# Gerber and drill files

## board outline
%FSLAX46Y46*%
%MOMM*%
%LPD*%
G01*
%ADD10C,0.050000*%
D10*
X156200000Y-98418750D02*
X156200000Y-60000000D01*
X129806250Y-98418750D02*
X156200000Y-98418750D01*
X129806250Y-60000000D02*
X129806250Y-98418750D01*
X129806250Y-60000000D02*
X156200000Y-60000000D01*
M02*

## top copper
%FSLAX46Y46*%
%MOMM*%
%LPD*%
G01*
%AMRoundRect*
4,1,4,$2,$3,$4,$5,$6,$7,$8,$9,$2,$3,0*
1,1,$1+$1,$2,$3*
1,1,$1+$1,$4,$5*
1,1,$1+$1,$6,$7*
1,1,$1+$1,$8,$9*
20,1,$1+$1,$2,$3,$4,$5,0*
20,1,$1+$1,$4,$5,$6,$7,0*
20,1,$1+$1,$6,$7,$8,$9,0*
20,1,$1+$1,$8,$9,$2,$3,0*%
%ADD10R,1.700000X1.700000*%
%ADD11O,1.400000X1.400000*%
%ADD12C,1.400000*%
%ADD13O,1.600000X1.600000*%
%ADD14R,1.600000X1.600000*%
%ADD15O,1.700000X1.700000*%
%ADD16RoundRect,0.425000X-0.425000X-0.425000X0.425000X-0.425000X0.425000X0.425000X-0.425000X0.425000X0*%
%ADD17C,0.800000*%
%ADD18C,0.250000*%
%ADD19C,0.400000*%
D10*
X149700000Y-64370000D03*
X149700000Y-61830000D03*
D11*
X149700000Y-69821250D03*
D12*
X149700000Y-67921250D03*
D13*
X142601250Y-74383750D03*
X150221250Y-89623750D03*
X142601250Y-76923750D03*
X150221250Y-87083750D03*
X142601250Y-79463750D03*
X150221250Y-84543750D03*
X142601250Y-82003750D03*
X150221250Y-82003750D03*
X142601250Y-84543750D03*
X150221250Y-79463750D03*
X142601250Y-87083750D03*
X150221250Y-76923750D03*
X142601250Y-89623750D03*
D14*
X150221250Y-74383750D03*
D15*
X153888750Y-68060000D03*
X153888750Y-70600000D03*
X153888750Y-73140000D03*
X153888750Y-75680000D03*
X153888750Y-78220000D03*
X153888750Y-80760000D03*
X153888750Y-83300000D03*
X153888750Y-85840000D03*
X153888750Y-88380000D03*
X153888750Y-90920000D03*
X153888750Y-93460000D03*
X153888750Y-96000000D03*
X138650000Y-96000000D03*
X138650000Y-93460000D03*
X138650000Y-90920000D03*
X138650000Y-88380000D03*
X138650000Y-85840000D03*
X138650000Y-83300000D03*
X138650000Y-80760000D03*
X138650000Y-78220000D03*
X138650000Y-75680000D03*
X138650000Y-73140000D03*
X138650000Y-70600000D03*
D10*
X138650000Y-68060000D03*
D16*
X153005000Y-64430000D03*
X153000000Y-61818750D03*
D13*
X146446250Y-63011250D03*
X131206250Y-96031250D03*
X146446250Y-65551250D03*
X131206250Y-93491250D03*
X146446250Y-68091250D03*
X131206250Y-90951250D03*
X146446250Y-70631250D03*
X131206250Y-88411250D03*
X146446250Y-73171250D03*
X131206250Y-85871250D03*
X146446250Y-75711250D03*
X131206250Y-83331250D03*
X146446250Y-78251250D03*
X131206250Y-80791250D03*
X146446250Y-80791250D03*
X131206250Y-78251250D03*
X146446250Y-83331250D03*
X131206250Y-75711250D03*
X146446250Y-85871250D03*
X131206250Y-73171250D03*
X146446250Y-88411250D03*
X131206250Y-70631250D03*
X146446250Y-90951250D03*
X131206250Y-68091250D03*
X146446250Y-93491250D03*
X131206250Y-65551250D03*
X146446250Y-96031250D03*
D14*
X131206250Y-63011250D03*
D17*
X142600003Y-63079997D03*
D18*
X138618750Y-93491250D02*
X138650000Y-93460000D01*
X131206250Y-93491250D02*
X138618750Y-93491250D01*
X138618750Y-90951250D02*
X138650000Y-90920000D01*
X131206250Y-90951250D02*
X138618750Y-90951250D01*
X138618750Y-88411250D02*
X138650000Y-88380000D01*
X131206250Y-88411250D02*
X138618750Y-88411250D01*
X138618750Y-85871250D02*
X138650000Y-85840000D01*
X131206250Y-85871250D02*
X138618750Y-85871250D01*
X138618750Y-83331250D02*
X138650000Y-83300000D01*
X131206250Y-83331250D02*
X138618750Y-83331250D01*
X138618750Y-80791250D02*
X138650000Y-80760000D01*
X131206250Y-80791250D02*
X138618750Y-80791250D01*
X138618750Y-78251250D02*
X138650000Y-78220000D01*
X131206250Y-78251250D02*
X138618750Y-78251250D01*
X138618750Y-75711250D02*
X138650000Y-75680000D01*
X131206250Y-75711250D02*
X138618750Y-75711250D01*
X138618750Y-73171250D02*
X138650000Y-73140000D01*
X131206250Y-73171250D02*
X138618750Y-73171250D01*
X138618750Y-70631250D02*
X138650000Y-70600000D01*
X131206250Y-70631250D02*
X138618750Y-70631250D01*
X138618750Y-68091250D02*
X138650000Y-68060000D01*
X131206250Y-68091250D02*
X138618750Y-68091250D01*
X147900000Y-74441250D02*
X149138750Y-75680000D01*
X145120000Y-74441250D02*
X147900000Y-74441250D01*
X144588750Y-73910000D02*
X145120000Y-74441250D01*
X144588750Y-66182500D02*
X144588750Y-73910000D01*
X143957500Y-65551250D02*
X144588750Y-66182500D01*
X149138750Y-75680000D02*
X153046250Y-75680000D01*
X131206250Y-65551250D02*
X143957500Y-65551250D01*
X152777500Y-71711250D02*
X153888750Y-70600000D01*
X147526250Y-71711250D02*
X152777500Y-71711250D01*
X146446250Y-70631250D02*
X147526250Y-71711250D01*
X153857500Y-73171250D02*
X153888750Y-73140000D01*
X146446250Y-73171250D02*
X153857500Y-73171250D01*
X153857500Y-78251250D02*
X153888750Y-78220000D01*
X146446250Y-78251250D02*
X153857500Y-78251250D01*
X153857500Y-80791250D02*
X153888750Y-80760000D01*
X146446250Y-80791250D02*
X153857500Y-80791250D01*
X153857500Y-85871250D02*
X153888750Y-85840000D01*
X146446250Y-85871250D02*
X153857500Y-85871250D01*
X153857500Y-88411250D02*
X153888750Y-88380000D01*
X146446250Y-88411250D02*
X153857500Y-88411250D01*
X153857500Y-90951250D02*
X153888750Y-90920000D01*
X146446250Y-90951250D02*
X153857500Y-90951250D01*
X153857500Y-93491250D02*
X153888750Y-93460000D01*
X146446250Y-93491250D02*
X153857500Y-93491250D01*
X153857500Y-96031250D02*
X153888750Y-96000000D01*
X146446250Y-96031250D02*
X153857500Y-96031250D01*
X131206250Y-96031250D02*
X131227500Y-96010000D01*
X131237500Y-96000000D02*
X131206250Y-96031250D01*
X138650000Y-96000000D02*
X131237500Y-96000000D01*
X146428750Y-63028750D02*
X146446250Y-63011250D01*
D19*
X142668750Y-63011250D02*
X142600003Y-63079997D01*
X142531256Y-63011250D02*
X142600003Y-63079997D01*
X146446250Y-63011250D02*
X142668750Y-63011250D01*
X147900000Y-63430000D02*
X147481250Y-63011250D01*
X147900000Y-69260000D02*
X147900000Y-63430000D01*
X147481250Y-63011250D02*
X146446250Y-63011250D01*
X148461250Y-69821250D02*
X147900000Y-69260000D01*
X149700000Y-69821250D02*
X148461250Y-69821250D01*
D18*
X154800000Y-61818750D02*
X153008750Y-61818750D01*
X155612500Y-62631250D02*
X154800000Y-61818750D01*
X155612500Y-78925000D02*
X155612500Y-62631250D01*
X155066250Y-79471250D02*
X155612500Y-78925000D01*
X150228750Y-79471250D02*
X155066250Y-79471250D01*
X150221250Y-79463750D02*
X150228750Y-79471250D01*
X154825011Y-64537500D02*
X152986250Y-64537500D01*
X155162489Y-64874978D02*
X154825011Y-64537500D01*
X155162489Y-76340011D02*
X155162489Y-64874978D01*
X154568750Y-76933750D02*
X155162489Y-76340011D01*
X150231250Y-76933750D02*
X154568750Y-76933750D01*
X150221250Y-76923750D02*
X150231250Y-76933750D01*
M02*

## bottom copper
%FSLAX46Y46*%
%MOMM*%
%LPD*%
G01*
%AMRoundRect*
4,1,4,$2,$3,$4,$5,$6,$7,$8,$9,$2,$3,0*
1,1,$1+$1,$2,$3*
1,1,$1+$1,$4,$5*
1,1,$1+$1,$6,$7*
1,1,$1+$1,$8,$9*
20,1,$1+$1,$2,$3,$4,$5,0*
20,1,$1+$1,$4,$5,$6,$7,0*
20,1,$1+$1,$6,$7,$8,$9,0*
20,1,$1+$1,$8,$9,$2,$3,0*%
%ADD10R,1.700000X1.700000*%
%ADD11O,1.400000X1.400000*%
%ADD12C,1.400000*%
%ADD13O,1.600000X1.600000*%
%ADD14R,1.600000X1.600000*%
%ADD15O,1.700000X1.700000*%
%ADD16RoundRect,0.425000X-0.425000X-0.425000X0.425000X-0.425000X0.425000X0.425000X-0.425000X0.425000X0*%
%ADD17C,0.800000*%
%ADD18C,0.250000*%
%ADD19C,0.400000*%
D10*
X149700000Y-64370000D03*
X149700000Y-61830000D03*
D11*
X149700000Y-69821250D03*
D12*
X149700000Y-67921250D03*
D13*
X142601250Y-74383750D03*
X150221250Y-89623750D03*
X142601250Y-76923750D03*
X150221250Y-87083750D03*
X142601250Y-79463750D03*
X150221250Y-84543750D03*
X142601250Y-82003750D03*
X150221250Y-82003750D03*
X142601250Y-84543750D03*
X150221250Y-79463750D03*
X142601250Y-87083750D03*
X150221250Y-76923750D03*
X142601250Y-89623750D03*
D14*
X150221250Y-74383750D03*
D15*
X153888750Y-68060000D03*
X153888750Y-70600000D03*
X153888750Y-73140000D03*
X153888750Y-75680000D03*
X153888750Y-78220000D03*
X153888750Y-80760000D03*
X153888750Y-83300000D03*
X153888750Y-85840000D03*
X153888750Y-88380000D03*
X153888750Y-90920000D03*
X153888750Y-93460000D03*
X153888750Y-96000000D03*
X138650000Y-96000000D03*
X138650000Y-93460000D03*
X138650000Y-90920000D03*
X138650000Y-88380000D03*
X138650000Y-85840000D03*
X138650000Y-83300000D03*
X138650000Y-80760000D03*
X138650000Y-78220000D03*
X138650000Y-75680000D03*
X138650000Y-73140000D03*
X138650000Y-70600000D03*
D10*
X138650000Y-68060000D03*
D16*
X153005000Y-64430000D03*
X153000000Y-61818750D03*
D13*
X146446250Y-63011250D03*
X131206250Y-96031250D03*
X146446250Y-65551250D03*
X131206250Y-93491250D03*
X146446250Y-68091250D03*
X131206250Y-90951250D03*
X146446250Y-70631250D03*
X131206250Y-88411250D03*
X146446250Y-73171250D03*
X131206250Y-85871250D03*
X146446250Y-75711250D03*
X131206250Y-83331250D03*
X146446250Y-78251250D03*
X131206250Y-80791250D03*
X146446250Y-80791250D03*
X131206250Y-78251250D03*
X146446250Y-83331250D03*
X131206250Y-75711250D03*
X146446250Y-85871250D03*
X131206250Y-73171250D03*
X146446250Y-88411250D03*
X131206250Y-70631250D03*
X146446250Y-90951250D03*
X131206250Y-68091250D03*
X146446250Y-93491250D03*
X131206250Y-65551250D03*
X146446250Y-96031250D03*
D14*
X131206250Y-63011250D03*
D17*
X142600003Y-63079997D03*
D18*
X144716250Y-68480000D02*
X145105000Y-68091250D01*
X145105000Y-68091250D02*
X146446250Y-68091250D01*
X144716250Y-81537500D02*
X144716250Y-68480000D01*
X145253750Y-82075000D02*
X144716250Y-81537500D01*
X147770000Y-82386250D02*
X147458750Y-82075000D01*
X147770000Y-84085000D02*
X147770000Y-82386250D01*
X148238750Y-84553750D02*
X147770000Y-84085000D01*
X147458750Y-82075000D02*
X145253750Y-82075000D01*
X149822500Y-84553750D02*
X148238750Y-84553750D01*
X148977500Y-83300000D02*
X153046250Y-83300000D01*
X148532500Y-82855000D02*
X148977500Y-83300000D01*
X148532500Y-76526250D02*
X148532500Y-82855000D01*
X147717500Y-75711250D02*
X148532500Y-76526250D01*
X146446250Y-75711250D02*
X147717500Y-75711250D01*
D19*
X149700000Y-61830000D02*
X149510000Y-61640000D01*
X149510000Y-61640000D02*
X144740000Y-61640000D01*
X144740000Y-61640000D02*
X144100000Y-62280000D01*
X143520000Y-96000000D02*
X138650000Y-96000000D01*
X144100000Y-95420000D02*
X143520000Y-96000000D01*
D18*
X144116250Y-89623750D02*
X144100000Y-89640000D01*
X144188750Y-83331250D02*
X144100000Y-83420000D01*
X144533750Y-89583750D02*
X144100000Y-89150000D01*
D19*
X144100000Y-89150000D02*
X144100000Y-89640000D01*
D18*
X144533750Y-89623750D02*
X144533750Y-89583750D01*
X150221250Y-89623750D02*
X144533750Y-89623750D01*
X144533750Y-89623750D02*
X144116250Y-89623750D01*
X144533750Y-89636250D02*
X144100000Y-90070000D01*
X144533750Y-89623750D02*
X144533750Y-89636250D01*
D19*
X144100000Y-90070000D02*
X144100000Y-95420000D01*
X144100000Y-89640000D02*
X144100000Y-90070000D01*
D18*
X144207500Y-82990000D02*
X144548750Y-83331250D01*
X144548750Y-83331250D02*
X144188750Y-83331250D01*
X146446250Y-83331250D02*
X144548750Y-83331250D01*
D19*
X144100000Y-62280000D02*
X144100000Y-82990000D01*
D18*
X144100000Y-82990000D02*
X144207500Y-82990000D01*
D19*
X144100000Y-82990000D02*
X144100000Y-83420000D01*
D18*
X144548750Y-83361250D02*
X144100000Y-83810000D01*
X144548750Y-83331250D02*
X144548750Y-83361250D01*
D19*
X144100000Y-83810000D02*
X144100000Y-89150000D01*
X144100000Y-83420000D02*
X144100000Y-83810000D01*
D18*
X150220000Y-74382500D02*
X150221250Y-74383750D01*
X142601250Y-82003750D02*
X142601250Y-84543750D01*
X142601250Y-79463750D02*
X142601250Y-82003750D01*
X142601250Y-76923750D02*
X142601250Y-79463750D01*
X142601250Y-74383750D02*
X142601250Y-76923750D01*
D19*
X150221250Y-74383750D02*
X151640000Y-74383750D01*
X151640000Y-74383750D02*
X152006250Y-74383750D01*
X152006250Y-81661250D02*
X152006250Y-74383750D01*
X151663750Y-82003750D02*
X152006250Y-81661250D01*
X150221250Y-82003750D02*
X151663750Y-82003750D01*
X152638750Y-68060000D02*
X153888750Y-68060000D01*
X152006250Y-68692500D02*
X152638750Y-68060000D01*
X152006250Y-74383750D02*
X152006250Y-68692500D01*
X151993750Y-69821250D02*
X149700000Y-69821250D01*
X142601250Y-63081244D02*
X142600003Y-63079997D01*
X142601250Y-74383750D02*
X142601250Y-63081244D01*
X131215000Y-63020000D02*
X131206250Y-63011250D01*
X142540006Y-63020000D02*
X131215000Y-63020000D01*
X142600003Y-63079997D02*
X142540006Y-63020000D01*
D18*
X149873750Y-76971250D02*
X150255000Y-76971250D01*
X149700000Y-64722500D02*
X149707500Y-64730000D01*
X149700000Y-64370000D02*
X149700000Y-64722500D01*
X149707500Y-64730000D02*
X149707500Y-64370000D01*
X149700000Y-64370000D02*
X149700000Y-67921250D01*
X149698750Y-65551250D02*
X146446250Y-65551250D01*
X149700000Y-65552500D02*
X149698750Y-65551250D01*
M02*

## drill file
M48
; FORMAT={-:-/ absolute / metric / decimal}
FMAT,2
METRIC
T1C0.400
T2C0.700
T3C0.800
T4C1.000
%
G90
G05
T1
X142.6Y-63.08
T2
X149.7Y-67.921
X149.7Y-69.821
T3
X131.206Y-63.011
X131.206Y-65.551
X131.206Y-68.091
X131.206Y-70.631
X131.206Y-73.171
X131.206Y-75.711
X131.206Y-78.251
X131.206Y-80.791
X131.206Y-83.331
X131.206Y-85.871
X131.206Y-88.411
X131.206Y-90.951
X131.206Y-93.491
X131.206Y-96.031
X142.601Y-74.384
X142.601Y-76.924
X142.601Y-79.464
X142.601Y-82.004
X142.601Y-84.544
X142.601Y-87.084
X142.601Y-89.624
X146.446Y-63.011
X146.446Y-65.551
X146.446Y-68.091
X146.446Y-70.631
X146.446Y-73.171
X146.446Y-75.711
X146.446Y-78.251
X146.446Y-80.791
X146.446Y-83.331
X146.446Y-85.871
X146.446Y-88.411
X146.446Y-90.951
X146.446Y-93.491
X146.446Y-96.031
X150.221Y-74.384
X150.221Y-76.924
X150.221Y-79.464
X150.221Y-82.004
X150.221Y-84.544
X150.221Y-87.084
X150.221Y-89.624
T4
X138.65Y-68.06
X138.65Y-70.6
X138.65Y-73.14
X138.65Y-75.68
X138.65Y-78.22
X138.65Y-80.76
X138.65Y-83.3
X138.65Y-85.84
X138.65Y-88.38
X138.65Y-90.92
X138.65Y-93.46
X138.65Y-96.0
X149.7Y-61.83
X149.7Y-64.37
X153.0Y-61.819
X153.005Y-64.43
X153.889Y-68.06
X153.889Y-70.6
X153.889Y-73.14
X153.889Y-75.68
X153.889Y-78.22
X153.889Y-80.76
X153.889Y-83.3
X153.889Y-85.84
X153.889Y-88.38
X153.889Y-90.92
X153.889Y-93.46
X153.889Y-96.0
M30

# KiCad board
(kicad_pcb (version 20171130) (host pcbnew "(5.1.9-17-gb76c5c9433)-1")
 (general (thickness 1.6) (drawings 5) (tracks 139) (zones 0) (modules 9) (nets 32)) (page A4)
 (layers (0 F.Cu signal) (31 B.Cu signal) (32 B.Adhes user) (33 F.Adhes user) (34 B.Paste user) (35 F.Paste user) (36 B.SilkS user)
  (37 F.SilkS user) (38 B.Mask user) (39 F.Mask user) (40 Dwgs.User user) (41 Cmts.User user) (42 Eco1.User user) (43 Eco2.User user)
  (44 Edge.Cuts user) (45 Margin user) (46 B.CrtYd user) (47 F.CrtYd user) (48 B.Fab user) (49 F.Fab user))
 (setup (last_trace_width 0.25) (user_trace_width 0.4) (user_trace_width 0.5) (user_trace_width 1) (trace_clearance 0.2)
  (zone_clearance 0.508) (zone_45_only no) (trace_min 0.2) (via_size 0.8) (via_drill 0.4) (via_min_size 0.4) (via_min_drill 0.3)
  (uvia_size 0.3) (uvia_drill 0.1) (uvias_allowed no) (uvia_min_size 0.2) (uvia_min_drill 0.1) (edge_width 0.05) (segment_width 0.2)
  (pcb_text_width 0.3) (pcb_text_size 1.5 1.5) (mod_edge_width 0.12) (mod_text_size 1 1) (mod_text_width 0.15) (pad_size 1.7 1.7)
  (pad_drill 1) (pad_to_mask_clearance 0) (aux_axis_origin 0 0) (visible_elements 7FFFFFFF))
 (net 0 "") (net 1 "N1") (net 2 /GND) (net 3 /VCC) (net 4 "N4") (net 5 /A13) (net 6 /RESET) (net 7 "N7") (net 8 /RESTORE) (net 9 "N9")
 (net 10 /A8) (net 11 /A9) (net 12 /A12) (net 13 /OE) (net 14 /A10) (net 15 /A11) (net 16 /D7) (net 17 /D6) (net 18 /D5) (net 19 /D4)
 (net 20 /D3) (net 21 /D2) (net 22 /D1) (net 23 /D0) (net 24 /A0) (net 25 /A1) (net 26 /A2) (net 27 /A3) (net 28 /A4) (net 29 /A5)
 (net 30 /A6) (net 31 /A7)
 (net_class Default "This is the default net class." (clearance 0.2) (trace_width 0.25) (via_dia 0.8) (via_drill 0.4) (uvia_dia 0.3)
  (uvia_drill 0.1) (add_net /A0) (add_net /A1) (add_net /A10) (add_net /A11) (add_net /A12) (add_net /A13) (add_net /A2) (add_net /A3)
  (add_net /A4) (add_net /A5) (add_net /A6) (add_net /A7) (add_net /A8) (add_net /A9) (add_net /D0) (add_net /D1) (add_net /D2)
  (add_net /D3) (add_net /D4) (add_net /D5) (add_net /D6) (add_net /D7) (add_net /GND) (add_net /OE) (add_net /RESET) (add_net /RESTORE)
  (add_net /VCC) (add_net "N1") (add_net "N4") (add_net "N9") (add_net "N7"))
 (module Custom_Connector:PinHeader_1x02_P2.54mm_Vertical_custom (layer F.Cu) (at 149.7 61.83)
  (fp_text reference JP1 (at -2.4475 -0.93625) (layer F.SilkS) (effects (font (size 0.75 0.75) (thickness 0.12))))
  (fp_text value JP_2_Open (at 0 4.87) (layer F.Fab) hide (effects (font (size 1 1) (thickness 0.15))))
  (pad 2 thru_hole rect (at 0 2.54) (size 1.7 1.7) (drill 1) (layers *.Cu *.Mask) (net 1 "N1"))
  (pad 1 thru_hole rect (at 0 0) (size 1.7 1.7) (drill 1) (layers *.Cu *.Mask) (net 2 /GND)))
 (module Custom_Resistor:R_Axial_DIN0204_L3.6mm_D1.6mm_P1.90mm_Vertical (layer F.Cu) (at 149.7 67.92125 270)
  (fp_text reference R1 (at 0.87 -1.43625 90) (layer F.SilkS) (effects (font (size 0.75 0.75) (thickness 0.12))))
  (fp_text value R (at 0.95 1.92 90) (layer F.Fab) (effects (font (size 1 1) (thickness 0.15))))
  (pad 2 thru_hole oval (at 1.9 0 270) (size 1.4 1.4) (drill 0.7) (layers *.Cu *.Mask) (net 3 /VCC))
  (pad 1 thru_hole circle (at 0 0 270) (size 1.4 1.4) (drill 0.7) (layers *.Cu *.Mask) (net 1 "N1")))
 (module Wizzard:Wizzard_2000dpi (layer F.Cu) (at 138.17125 65.0425 350)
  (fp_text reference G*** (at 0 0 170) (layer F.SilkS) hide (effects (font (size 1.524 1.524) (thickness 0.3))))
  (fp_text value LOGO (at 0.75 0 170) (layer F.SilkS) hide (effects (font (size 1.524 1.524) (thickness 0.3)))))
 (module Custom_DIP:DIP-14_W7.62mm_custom (layer B.Cu) (at 150.22125 74.38375 180)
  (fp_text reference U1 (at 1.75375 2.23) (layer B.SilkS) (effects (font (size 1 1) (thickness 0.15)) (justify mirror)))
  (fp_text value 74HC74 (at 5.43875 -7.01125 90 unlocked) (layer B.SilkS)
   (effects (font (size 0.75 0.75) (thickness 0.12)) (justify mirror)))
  (pad 14 thru_hole oval (at 7.62 0 180) (size 1.6 1.6) (drill 0.8) (layers *.Cu *.Mask) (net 3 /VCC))
  (pad 7 thru_hole oval (at 0 -15.24 180) (size 1.6 1.6) (drill 0.8) (layers *.Cu *.Mask) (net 2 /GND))
  (pad 13 thru_hole oval (at 7.62 -2.54 180) (size 1.6 1.6) (drill 0.8) (layers *.Cu *.Mask) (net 3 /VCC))
  (pad 6 thru_hole oval (at 0 -12.7 180) (size 1.6 1.6) (drill 0.8) (layers *.Cu *.Mask) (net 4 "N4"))
  (pad 12 thru_hole oval (at 7.62 -5.08 180) (size 1.6 1.6) (drill 0.8) (layers *.Cu *.Mask) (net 3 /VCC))
  (pad 5 thru_hole oval (at 0 -10.16 180) (size 1.6 1.6) (drill 0.8) (layers *.Cu *.Mask) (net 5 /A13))
  (pad 11 thru_hole oval (at 7.62 -7.62 180) (size 1.6 1.6) (drill 0.8) (layers *.Cu *.Mask) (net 3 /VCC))
  (pad 4 thru_hole oval (at 0 -7.62 180) (size 1.6 1.6) (drill 0.8) (layers *.Cu *.Mask) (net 3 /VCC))
  (pad 10 thru_hole oval (at 7.62 -10.16 180) (size 1.6 1.6) (drill 0.8) (layers *.Cu *.Mask) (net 3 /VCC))
  (pad 3 thru_hole oval (at 0 -5.08 180) (size 1.6 1.6) (drill 0.8) (layers *.Cu *.Mask) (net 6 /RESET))
  (pad 9 thru_hole oval (at 7.62 -12.7 180) (size 1.6 1.6) (drill 0.8) (layers *.Cu *.Mask) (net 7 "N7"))
  (pad 2 thru_hole oval (at 0 -2.54 180) (size 1.6 1.6) (drill 0.8) (layers *.Cu *.Mask) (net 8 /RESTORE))
  (pad 8 thru_hole oval (at 7.62 -15.24 180) (size 1.6 1.6) (drill 0.8) (layers *.Cu *.Mask) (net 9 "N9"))
  (pad 1 thru_hole rect (at 0 0 180) (size 1.6 1.6) (drill 0.8) (layers *.Cu *.Mask) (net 3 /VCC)))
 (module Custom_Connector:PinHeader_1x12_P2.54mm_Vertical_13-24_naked (layer F.Cu) (at 153.88875 68.06)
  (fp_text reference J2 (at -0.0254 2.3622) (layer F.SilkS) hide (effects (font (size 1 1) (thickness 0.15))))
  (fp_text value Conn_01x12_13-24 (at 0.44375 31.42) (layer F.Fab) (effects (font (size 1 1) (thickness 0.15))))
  (pad 24 thru_hole oval (at 0 0) (size 1.7 1.7) (drill 1) (layers *.Cu *.Mask) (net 3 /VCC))
  (pad 23 thru_hole oval (at 0 2.54) (size 1.7 1.7) (drill 1) (layers *.Cu *.Mask) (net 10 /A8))
  (pad 22 thru_hole oval (at 0 5.08) (size 1.7 1.7) (drill 1) (layers *.Cu *.Mask) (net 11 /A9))
  (pad 21 thru_hole oval (at 0 7.62) (size 1.7 1.7) (drill 1) (layers *.Cu *.Mask) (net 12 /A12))
  (pad 20 thru_hole oval (at 0 10.16) (size 1.7 1.7) (drill 1) (layers *.Cu *.Mask) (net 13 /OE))
  (pad 19 thru_hole oval (at 0 12.7) (size 1.7 1.7) (drill 1) (layers *.Cu *.Mask) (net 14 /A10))
  (pad 18 thru_hole oval (at 0 15.24) (size 1.7 1.7) (drill 1) (layers *.Cu *.Mask) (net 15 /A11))
  (pad 17 thru_hole oval (at 0 17.78) (size 1.7 1.7) (drill 1) (layers *.Cu *.Mask) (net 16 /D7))
  (pad 16 thru_hole oval (at 0 20.32) (size 1.7 1.7) (drill 1) (layers *.Cu *.Mask) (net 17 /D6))
  (pad 15 thru_hole oval (at 0 22.86) (size 1.7 1.7) (drill 1) (layers *.Cu *.Mask) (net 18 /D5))
  (pad 14 thru_hole oval (at 0 25.4) (size 1.7 1.7) (drill 1) (layers *.Cu *.Mask) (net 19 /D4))
  (pad 13 thru_hole oval (at 0 27.94) (size 1.7 1.7) (drill 1) (layers *.Cu *.Mask) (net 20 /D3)))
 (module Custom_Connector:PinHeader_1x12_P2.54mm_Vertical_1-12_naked (layer F.Cu) (at 138.65 68.06)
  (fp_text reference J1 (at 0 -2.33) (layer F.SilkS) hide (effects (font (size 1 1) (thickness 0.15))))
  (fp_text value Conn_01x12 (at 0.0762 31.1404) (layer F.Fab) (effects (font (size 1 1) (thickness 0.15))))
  (pad 12 thru_hole oval (at 0 27.94) (size 1.7 1.7) (drill 1) (layers *.Cu *.Mask) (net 2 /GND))
  (pad 11 thru_hole oval (at 0 25.4) (size 1.7 1.7) (drill 1) (layers *.Cu *.Mask) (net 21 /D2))
  (pad 10 thru_hole oval (at 0 22.86) (size 1.7 1.7) (drill 1) (layers *.Cu *.Mask) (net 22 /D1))
  (pad 9 thru_hole oval (at 0 20.32) (size 1.7 1.7) (drill 1) (layers *.Cu *.Mask) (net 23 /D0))
  (pad 8 thru_hole oval (at 0 17.78) (size 1.7 1.7) (drill 1) (layers *.Cu *.Mask) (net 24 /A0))
  (pad 7 thru_hole oval (at 0 15.24) (size 1.7 1.7) (drill 1) (layers *.Cu *.Mask) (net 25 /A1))
  (pad 6 thru_hole oval (at 0 12.7) (size 1.7 1.7) (drill 1) (layers *.Cu *.Mask) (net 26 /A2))
  (pad 5 thru_hole oval (at 0 10.16) (size 1.7 1.7) (drill 1) (layers *.Cu *.Mask) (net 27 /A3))
  (pad 4 thru_hole oval (at 0 7.62) (size 1.7 1.7) (drill 1) (layers *.Cu *.Mask) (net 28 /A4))
  (pad 3 thru_hole oval (at 0 5.08) (size 1.7 1.7) (drill 1) (layers *.Cu *.Mask) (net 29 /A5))
  (pad 2 thru_hole oval (at 0 2.54) (size 1.7 1.7) (drill 1) (layers *.Cu *.Mask) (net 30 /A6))
  (pad 1 thru_hole rect (at 0 0) (size 1.7 1.7) (drill 1) (layers *.Cu *.Mask) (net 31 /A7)))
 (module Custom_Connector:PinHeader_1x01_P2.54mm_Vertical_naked (layer F.Cu) (at 153.02 64.43)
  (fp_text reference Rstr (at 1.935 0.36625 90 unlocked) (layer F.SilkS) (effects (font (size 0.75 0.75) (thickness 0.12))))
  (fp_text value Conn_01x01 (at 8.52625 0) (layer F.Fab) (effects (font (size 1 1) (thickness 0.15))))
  (pad 1 thru_hole roundrect (at -0.015 0) (size 1.7 1.7) (drill 1) (layers *.Cu *.Mask) (roundrect_rratio 0.25) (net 8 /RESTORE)))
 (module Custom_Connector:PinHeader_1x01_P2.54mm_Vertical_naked (layer F.Cu) (at 153.0175 61.81875)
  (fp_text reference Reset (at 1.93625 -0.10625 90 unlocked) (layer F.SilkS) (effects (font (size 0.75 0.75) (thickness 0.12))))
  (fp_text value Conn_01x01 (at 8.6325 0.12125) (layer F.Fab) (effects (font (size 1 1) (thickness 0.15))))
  (pad 1 thru_hole roundrect (at -0.0175 0) (size 1.7 1.7) (drill 1) (layers *.Cu *.Mask) (roundrect_rratio 0.25) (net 6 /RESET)))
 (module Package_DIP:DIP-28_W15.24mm (layer F.Cu) (at 131.20625 63.01125)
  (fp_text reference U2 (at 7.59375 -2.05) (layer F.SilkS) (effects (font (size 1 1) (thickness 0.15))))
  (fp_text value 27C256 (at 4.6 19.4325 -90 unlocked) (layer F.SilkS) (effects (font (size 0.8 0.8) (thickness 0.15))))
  (pad 28 thru_hole oval (at 15.24 0) (size 1.6 1.6) (drill 0.8) (layers *.Cu *.Mask) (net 3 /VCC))
  (pad 14 thru_hole oval (at 0 33.02) (size 1.6 1.6) (drill 0.8) (layers *.Cu *.Mask) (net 2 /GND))
  (pad 27 thru_hole oval (at 15.24 2.54) (size 1.6 1.6) (drill 0.8) (layers *.Cu *.Mask) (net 1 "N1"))
  (pad 13 thru_hole oval (at 0 30.48) (size 1.6 1.6) (drill 0.8) (layers *.Cu *.Mask) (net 21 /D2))
  (pad 26 thru_hole oval (at 15.24 5.08) (size 1.6 1.6) (drill 0.8) (layers *.Cu *.Mask) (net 5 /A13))
  (pad 12 thru_hole oval (at 0 27.94) (size 1.6 1.6) (drill 0.8) (layers *.Cu *.Mask) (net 22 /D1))
  (pad 25 thru_hole oval (at 15.24 7.62) (size 1.6 1.6) (drill 0.8) (layers *.Cu *.Mask) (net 10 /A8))
  (pad 11 thru_hole oval (at 0 25.4) (size 1.6 1.6) (drill 0.8) (layers *.Cu *.Mask) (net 23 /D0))
  (pad 24 thru_hole oval (at 15.24 10.16) (size 1.6 1.6) (drill 0.8) (layers *.Cu *.Mask) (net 11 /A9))
  (pad 10 thru_hole oval (at 0 22.86) (size 1.6 1.6) (drill 0.8) (layers *.Cu *.Mask) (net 24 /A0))
  (pad 23 thru_hole oval (at 15.24 12.7) (size 1.6 1.6) (drill 0.8) (layers *.Cu *.Mask) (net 15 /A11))
  (pad 9 thru_hole oval (at 0 20.32) (size 1.6 1.6) (drill 0.8) (layers *.Cu *.Mask) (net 25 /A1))
  (pad 22 thru_hole oval (at 15.24 15.24) (size 1.6 1.6) (drill 0.8) (layers *.Cu *.Mask) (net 13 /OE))
  (pad 8 thru_hole oval (at 0 17.78) (size 1.6 1.6) (drill 0.8) (layers *.Cu *.Mask) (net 26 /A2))
  (pad 21 thru_hole oval (at 15.24 17.78) (size 1.6 1.6) (drill 0.8) (layers *.Cu *.Mask) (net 14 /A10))
  (pad 7 thru_hole oval (at 0 15.24) (size 1.6 1.6) (drill 0.8) (layers *.Cu *.Mask) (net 27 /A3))
  (pad 20 thru_hole oval (at 15.24 20.32) (size 1.6 1.6) (drill 0.8) (layers *.Cu *.Mask) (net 2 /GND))
  (pad 6 thru_hole oval (at 0 12.7) (size 1.6 1.6) (drill 0.8) (layers *.Cu *.Mask) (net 28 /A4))
  (pad 19 thru_hole oval (at 15.24 22.86) (size 1.6 1.6) (drill 0.8) (layers *.Cu *.Mask) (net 16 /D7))
  (pad 5 thru_hole oval (at 0 10.16) (size 1.6 1.6) (drill 0.8) (layers *.Cu *.Mask) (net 29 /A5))
  (pad 18 thru_hole oval (at 15.24 25.4) (size 1.6 1.6) (drill 0.8) (layers *.Cu *.Mask) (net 17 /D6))
  (pad 4 thru_hole oval (at 0 7.62) (size 1.6 1.6) (drill 0.8) (layers *.Cu *.Mask) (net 30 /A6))
  (pad 17 thru_hole oval (at 15.24 27.94) (size 1.6 1.6) (drill 0.8) (layers *.Cu *.Mask) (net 18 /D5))
  (pad 3 thru_hole oval (at 0 5.08) (size 1.6 1.6) (drill 0.8) (layers *.Cu *.Mask) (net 31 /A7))
  (pad 16 thru_hole oval (at 15.24 30.48) (size 1.6 1.6) (drill 0.8) (layers *.Cu *.Mask) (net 19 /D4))
  (pad 2 thru_hole oval (at 0 2.54) (size 1.6 1.6) (drill 0.8) (layers *.Cu *.Mask) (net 12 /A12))
  (pad 15 thru_hole oval (at 15.24 33.02) (size 1.6 1.6) (drill 0.8) (layers *.Cu *.Mask) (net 20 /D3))
  (pad 1 thru_hole rect (at 0 0) (size 1.6 1.6) (drill 0.8) (layers *.Cu *.Mask) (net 3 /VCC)))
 (gr_line (start 156.2 98.41875) (end 156.2 60) (layer Edge.Cuts) (width 0.05))
 (gr_line (start 129.80625 98.41875) (end 156.2 98.41875) (layer Edge.Cuts) (width 0.05))
 (gr_line (start 129.80625 60) (end 129.80625 98.41875) (layer Edge.Cuts) (width 0.05))
 (gr_line (start 129.80625 60) (end 156.2 60) (layer Edge.Cuts) (width 0.05))
 (segment (start 138.61875 93.49125) (end 138.65 93.46) (width 0.25) (layer F.Cu) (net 21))
 (segment (start 131.20625 93.49125) (end 138.61875 93.49125) (width 0.25) (layer F.Cu) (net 21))
 (segment (start 138.61875 90.95125) (end 138.65 90.92) (width 0.25) (layer F.Cu) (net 22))
 (segment (start 131.20625 90.95125) (end 138.61875 90.95125) (width 0.25) (layer F.Cu) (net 22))
 (segment (start 138.61875 88.41125) (end 138.65 88.38) (width 0.25) (layer F.Cu) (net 23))
 (segment (start 131.20625 88.41125) (end 138.61875 88.41125) (width 0.25) (layer F.Cu) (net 23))
 (segment (start 138.61875 85.87125) (end 138.65 85.84) (width 0.25) (layer F.Cu) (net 24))
 (segment (start 131.20625 85.87125) (end 138.61875 85.87125) (width 0.25) (layer F.Cu) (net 24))
 (segment (start 138.61875 83.33125) (end 138.65 83.3) (width 0.25) (layer F.Cu) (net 25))
 (segment (start 131.20625 83.33125) (end 138.61875 83.33125) (width 0.25) (layer F.Cu) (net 25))
 (segment (start 138.61875 80.79125) (end 138.65 80.76) (width 0.25) (layer F.Cu) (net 26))
 (segment (start 131.20625 80.79125) (end 138.61875 80.79125) (width 0.25) (layer F.Cu) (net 26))
 (segment (start 138.61875 78.25125) (end 138.65 78.22) (width 0.25) (layer F.Cu) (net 27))
 (segment (start 131.20625 78.25125) (end 138.61875 78.25125) (width 0.25) (layer F.Cu) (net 27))
 (segment (start 138.61875 75.71125) (end 138.65 75.68) (width 0.25) (layer F.Cu) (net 28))
 (segment (start 131.20625 75.71125) (end 138.61875 75.71125) (width 0.25) (layer F.Cu) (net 28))
 (segment (start 138.61875 73.17125) (end 138.65 73.14) (width 0.25) (layer F.Cu) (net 29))
 (segment (start 131.20625 73.17125) (end 138.61875 73.17125) (width 0.25) (layer F.Cu) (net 29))
 (segment (start 138.61875 70.63125) (end 138.65 70.6) (width 0.25) (layer F.Cu) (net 30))
 (segment (start 131.20625 70.63125) (end 138.61875 70.63125) (width 0.25) (layer F.Cu) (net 30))
 (segment (start 138.61875 68.09125) (end 138.65 68.06) (width 0.25) (layer F.Cu) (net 31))
 (segment (start 131.20625 68.09125) (end 138.61875 68.09125) (width 0.25) (layer F.Cu) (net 31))
 (segment (start 147.9 74.44125) (end 149.13875 75.68) (width 0.25) (layer F.Cu) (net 12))
 (segment (start 145.12 74.44125) (end 147.9 74.44125) (width 0.25) (layer F.Cu) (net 12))
 (segment (start 144.58875 73.91) (end 145.12 74.44125) (width 0.25) (layer F.Cu) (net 12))
 (segment (start 144.58875 66.1825) (end 144.58875 73.91) (width 0.25) (layer F.Cu) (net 12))
 (segment (start 143.9575 65.55125) (end 144.58875 66.1825) (width 0.25) (layer F.Cu) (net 12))
 (segment (start 149.13875 75.68) (end 153.04625 75.68) (width 0.25) (layer F.Cu) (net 12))
 (segment (start 131.20625 65.55125) (end 143.9575 65.55125) (width 0.25) (layer F.Cu) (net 12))
 (segment (start 144.71625 68.48) (end 145.105 68.09125) (width 0.25) (layer B.Cu) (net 5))
 (segment (start 145.105 68.09125) (end 146.44625 68.09125) (width 0.25) (layer B.Cu) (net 5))
 (segment (start 144.71625 81.5375) (end 144.71625 68.48) (width 0.25) (layer B.Cu) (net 5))
 (segment (start 145.25375 82.075) (end 144.71625 81.5375) (width 0.25) (layer B.Cu) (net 5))
 (segment (start 147.77 82.38625) (end 147.45875 82.075) (width 0.25) (layer B.Cu) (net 5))
 (segment (start 147.77 84.085) (end 147.77 82.38625) (width 0.25) (layer B.Cu) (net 5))
 (segment (start 148.23875 84.55375) (end 147.77 84.085) (width 0.25) (layer B.Cu) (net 5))
 (segment (start 147.45875 82.075) (end 145.25375 82.075) (width 0.25) (layer B.Cu) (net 5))
 (segment (start 149.8225 84.55375) (end 148.23875 84.55375) (width 0.25) (layer B.Cu) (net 5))
 (segment (start 152.7775 71.71125) (end 153.88875 70.6) (width 0.25) (layer F.Cu) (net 10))
 (segment (start 147.52625 71.71125) (end 152.7775 71.71125) (width 0.25) (layer F.Cu) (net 10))
 (segment (start 146.44625 70.63125) (end 147.52625 71.71125) (width 0.25) (layer F.Cu) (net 10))
 (segment (start 153.8575 73.17125) (end 153.88875 73.14) (width 0.25) (layer F.Cu) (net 11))
 (segment (start 146.44625 73.17125) (end 153.8575 73.17125) (width 0.25) (layer F.Cu) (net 11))
 (segment (start 148.9775 83.3) (end 153.04625 83.3) (width 0.25) (layer B.Cu) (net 15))
 (segment (start 148.5325 82.855) (end 148.9775 83.3) (width 0.25) (layer B.Cu) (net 15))
 (segment (start 148.5325 76.52625) (end 148.5325 82.855) (width 0.25) (layer B.Cu) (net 15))
 (segment (start 147.7175 75.71125) (end 148.5325 76.52625) (width 0.25) (layer B.Cu) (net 15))
 (segment (start 146.44625 75.71125) (end 147.7175 75.71125) (width 0.25) (layer B.Cu) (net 15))
 (segment (start 153.8575 78.25125) (end 153.88875 78.22) (width 0.25) (layer F.Cu) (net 13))
 (segment (start 146.44625 78.25125) (end 153.8575 78.25125) (width 0.25) (layer F.Cu) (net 13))
 (segment (start 153.8575 80.79125) (end 153.88875 80.76) (width 0.25) (layer F.Cu) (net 14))
 (segment (start 146.44625 80.79125) (end 153.8575 80.79125) (width 0.25) (layer F.Cu) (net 14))
 (segment (start 153.8575 85.87125) (end 153.88875 85.84) (width 0.25) (layer F.Cu) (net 16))
 (segment (start 146.44625 85.87125) (end 153.8575 85.87125) (width 0.25) (layer F.Cu) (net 16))
 (segment (start 153.8575 88.41125) (end 153.88875 88.38) (width 0.25) (layer F.Cu) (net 17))
 (segment (start 146.44625 88.41125) (end 153.8575 88.41125) (width 0.25) (layer F.Cu) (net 17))
 (segment (start 153.8575 90.95125) (end 153.88875 90.92) (width 0.25) (layer F.Cu) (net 18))
 (segment (start 146.44625 90.95125) (end 153.8575 90.95125) (width 0.25) (layer F.Cu) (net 18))
 (segment (start 153.8575 93.49125) (end 153.88875 93.46) (width 0.25) (layer F.Cu) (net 19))
 (segment (start 146.44625 93.49125) (end 153.8575 93.49125) (width 0.25) (layer F.Cu) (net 19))
 (segment (start 153.8575 96.03125) (end 153.88875 96) (width 0.25) (layer F.Cu) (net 20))
 (segment (start 146.44625 96.03125) (end 153.8575 96.03125) (width 0.25) (layer F.Cu) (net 20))
 (segment (start 131.20625 96.03125) (end 131.2275 96.01) (width 0.25) (layer F.Cu) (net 2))
 (segment (start 131.2375 96) (end 131.20625 96.03125) (width 0.25) (layer F.Cu) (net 2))
 (segment (start 138.65 96) (end 131.2375 96) (width 0.25) (layer F.Cu) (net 2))
 (segment (start 149.7 61.83) (end 149.51 61.64) (width 0.4) (layer B.Cu) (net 2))
 (segment (start 149.51 61.64) (end 144.74 61.64) (width 0.4) (layer B.Cu) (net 2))
 (segment (start 144.74 61.64) (end 144.1 62.28) (width 0.4) (layer B.Cu) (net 2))
 (segment (start 143.52 96) (end 138.65 96) (width 0.4) (layer B.Cu) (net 2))
 (segment (start 144.1 95.42) (end 143.52 96) (width 0.4) (layer B.Cu) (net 2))
 (segment (start 144.11625 89.62375) (end 144.1 89.64) (width 0.25) (layer B.Cu) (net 2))
 (segment (start 144.18875 83.33125) (end 144.1 83.42) (width 0.25) (layer B.Cu) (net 2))
 (segment (start 144.53375 89.58375) (end 144.1 89.15) (width 0.25) (layer B.Cu) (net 2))
 (segment (start 144.1 89.15) (end 144.1 89.64) (width 0.4) (layer B.Cu) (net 2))
 (segment (start 144.53375 89.62375) (end 144.53375 89.58375) (width 0.25) (layer B.Cu) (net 2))
 (segment (start 150.22125 89.62375) (end 144.53375 89.62375) (width 0.25) (layer B.Cu) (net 2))
 (segment (start 144.53375 89.62375) (end 144.11625 89.62375) (width 0.25) (layer B.Cu) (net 2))
 (segment (start 144.53375 89.63625) (end 144.1 90.07) (width 0.25) (layer B.Cu) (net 2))
 (segment (start 144.53375 89.62375) (end 144.53375 89.63625) (width 0.25) (layer B.Cu) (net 2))
 (segment (start 144.1 90.07) (end 144.1 95.42) (width 0.4) (layer B.Cu) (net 2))
 (segment (start 144.1 89.64) (end 144.1 90.07) (width 0.4) (layer B.Cu) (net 2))
 (segment (start 144.2075 82.99) (end 144.54875 83.33125) (width 0.25) (layer B.Cu) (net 2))
 (segment (start 144.54875 83.33125) (end 144.18875 83.33125) (width 0.25) (layer B.Cu) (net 2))
 (segment (start 146.44625 83.33125) (end 144.54875 83.33125) (width 0.25) (layer B.Cu) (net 2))
 (segment (start 144.1 62.28) (end 144.1 82.99) (width 0.4) (layer B.Cu) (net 2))
 (segment (start 144.1 82.99) (end 144.2075 82.99) (width 0.25) (layer B.Cu) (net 2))
 (segment (start 144.1 82.99) (end 144.1 83.42) (width 0.4) (layer B.Cu) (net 2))
 (segment (start 144.54875 83.36125) (end 144.1 83.81) (width 0.25) (layer B.Cu) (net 2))
 (segment (start 144.54875 83.33125) (end 144.54875 83.36125) (width 0.25) (layer B.Cu) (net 2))
 (segment (start 144.1 83.81) (end 144.1 89.15) (width 0.4) (layer B.Cu) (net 2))
 (segment (start 144.1 83.42) (end 144.1 83.81) (width 0.4) (layer B.Cu) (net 2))
 (segment (start 150.22 74.3825) (end 150.22125 74.38375) (width 0.25) (layer B.Cu) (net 3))
 (segment (start 146.42875 63.02875) (end 146.44625 63.01125) (width 0.25) (layer F.Cu) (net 3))
 (segment (start 142.60125 82.00375) (end 142.60125 84.54375) (width 0.25) (layer B.Cu) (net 3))
 (segment (start 142.60125 79.46375) (end 142.60125 82.00375) (width 0.25) (layer B.Cu) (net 3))
 (segment (start 142.60125 76.92375) (end 142.60125 79.46375) (width 0.25) (layer B.Cu) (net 3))
 (segment (start 142.60125 74.38375) (end 142.60125 76.92375) (width 0.25) (layer B.Cu) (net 3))
 (segment (start 150.22125 74.38375) (end 151.64 74.38375) (width 0.4) (layer B.Cu) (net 3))
 (segment (start 151.64 74.38375) (end 152.00625 74.38375) (width 0.4) (layer B.Cu) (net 3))
 (segment (start 152.00625 81.66125) (end 152.00625 74.38375) (width 0.4) (layer B.Cu) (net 3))
 (segment (start 151.66375 82.00375) (end 152.00625 81.66125) (width 0.4) (layer B.Cu) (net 3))
 (segment (start 150.22125 82.00375) (end 151.66375 82.00375) (width 0.4) (layer B.Cu) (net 3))
 (segment (start 152.63875 68.06) (end 153.88875 68.06) (width 0.4) (layer B.Cu) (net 3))
 (segment (start 152.00625 68.6925) (end 152.63875 68.06) (width 0.4) (layer B.Cu) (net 3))
 (segment (start 152.00625 74.38375) (end 152.00625 68.6925) (width 0.4) (layer B.Cu) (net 3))
 (segment (start 151.99375 69.82125) (end 149.7 69.82125) (width 0.4) (layer B.Cu) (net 3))
 (via (at 142.600003 63.079997) (size 0.8) (drill 0.4) (layers F.Cu B.Cu) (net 3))
 (segment (start 142.60125 63.081244) (end 142.600003 63.079997) (width 0.4) (layer B.Cu) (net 3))
 (segment (start 142.60125 74.38375) (end 142.60125 63.081244) (width 0.4) (layer B.Cu) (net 3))
 (segment (start 142.66875 63.01125) (end 142.600003 63.079997) (width 0.4) (layer F.Cu) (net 3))
 (segment (start 142.531256 63.01125) (end 142.600003 63.079997) (width 0.4) (layer F.Cu) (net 3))
 (segment (start 146.44625 63.01125) (end 142.66875 63.01125) (width 0.4) (layer F.Cu) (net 3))
 (segment (start 147.9 63.43) (end 147.48125 63.01125) (width 0.4) (layer F.Cu) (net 3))
 (segment (start 147.9 69.26) (end 147.9 63.43) (width 0.4) (layer F.Cu) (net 3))
 (segment (start 147.48125 63.01125) (end 146.44625 63.01125) (width 0.4) (layer F.Cu) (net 3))
 (segment (start 148.46125 69.82125) (end 147.9 69.26) (width 0.4) (layer F.Cu) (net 3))
 (segment (start 149.7 69.82125) (end 148.46125 69.82125) (width 0.4) (layer F.Cu) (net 3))
 (segment (start 131.215 63.02) (end 131.20625 63.01125) (width 0.4) (layer B.Cu) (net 3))
 (segment (start 142.540006 63.02) (end 131.215 63.02) (width 0.4) (layer B.Cu) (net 3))
 (segment (start 142.600003 63.079997) (end 142.540006 63.02) (width 0.4) (layer B.Cu) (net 3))
 (segment (start 154.8 61.81875) (end 153.00875 61.81875) (width 0.25) (layer F.Cu) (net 6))
 (segment (start 155.6125 62.63125) (end 154.8 61.81875) (width 0.25) (layer F.Cu) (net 6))
 (segment (start 155.6125 78.925) (end 155.6125 62.63125) (width 0.25) (layer F.Cu) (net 6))
 (segment (start 155.06625 79.47125) (end 155.6125 78.925) (width 0.25) (layer F.Cu) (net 6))
 (segment (start 150.22875 79.47125) (end 155.06625 79.47125) (width 0.25) (layer F.Cu) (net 6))
 (segment (start 150.22125 79.46375) (end 150.22875 79.47125) (width 0.25) (layer F.Cu) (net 6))
 (segment (start 149.87375 76.97125) (end 150.255 76.97125) (width 0.25) (layer B.Cu) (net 8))
 (segment (start 154.825011 64.5375) (end 152.98625 64.5375) (width 0.25) (layer F.Cu) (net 8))
 (segment (start 155.162489 64.874978) (end 154.825011 64.5375) (width 0.25) (layer F.Cu) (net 8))
 (segment (start 155.162489 76.340011) (end 155.162489 64.874978) (width 0.25) (layer F.Cu) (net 8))
 (segment (start 154.56875 76.93375) (end 155.162489 76.340011) (width 0.25) (layer F.Cu) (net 8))
 (segment (start 150.23125 76.93375) (end 154.56875 76.93375) (width 0.25) (layer F.Cu) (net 8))
 (segment (start 150.22125 76.92375) (end 150.23125 76.93375) (width 0.25) (layer F.Cu) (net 8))
 (segment (start 149.7 64.7225) (end 149.7075 64.73) (width 0.25) (layer B.Cu) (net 1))
 (segment (start 149.7 64.37) (end 149.7 64.7225) (width 0.25) (layer B.Cu) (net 1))
 (segment (start 149.7075 64.73) (end 149.7075 64.37) (width 0.25) (layer B.Cu) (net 1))
 (segment (start 149.7 64.37) (end 149.7 67.92125) (width 0.25) (layer B.Cu) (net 1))
 (segment (start 149.69875 65.55125) (end 146.44625 65.55125) (width 0.25) (layer B.Cu) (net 1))
 (segment (start 149.7 65.5525) (end 149.69875 65.55125) (width 0.25) (layer B.Cu) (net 1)))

